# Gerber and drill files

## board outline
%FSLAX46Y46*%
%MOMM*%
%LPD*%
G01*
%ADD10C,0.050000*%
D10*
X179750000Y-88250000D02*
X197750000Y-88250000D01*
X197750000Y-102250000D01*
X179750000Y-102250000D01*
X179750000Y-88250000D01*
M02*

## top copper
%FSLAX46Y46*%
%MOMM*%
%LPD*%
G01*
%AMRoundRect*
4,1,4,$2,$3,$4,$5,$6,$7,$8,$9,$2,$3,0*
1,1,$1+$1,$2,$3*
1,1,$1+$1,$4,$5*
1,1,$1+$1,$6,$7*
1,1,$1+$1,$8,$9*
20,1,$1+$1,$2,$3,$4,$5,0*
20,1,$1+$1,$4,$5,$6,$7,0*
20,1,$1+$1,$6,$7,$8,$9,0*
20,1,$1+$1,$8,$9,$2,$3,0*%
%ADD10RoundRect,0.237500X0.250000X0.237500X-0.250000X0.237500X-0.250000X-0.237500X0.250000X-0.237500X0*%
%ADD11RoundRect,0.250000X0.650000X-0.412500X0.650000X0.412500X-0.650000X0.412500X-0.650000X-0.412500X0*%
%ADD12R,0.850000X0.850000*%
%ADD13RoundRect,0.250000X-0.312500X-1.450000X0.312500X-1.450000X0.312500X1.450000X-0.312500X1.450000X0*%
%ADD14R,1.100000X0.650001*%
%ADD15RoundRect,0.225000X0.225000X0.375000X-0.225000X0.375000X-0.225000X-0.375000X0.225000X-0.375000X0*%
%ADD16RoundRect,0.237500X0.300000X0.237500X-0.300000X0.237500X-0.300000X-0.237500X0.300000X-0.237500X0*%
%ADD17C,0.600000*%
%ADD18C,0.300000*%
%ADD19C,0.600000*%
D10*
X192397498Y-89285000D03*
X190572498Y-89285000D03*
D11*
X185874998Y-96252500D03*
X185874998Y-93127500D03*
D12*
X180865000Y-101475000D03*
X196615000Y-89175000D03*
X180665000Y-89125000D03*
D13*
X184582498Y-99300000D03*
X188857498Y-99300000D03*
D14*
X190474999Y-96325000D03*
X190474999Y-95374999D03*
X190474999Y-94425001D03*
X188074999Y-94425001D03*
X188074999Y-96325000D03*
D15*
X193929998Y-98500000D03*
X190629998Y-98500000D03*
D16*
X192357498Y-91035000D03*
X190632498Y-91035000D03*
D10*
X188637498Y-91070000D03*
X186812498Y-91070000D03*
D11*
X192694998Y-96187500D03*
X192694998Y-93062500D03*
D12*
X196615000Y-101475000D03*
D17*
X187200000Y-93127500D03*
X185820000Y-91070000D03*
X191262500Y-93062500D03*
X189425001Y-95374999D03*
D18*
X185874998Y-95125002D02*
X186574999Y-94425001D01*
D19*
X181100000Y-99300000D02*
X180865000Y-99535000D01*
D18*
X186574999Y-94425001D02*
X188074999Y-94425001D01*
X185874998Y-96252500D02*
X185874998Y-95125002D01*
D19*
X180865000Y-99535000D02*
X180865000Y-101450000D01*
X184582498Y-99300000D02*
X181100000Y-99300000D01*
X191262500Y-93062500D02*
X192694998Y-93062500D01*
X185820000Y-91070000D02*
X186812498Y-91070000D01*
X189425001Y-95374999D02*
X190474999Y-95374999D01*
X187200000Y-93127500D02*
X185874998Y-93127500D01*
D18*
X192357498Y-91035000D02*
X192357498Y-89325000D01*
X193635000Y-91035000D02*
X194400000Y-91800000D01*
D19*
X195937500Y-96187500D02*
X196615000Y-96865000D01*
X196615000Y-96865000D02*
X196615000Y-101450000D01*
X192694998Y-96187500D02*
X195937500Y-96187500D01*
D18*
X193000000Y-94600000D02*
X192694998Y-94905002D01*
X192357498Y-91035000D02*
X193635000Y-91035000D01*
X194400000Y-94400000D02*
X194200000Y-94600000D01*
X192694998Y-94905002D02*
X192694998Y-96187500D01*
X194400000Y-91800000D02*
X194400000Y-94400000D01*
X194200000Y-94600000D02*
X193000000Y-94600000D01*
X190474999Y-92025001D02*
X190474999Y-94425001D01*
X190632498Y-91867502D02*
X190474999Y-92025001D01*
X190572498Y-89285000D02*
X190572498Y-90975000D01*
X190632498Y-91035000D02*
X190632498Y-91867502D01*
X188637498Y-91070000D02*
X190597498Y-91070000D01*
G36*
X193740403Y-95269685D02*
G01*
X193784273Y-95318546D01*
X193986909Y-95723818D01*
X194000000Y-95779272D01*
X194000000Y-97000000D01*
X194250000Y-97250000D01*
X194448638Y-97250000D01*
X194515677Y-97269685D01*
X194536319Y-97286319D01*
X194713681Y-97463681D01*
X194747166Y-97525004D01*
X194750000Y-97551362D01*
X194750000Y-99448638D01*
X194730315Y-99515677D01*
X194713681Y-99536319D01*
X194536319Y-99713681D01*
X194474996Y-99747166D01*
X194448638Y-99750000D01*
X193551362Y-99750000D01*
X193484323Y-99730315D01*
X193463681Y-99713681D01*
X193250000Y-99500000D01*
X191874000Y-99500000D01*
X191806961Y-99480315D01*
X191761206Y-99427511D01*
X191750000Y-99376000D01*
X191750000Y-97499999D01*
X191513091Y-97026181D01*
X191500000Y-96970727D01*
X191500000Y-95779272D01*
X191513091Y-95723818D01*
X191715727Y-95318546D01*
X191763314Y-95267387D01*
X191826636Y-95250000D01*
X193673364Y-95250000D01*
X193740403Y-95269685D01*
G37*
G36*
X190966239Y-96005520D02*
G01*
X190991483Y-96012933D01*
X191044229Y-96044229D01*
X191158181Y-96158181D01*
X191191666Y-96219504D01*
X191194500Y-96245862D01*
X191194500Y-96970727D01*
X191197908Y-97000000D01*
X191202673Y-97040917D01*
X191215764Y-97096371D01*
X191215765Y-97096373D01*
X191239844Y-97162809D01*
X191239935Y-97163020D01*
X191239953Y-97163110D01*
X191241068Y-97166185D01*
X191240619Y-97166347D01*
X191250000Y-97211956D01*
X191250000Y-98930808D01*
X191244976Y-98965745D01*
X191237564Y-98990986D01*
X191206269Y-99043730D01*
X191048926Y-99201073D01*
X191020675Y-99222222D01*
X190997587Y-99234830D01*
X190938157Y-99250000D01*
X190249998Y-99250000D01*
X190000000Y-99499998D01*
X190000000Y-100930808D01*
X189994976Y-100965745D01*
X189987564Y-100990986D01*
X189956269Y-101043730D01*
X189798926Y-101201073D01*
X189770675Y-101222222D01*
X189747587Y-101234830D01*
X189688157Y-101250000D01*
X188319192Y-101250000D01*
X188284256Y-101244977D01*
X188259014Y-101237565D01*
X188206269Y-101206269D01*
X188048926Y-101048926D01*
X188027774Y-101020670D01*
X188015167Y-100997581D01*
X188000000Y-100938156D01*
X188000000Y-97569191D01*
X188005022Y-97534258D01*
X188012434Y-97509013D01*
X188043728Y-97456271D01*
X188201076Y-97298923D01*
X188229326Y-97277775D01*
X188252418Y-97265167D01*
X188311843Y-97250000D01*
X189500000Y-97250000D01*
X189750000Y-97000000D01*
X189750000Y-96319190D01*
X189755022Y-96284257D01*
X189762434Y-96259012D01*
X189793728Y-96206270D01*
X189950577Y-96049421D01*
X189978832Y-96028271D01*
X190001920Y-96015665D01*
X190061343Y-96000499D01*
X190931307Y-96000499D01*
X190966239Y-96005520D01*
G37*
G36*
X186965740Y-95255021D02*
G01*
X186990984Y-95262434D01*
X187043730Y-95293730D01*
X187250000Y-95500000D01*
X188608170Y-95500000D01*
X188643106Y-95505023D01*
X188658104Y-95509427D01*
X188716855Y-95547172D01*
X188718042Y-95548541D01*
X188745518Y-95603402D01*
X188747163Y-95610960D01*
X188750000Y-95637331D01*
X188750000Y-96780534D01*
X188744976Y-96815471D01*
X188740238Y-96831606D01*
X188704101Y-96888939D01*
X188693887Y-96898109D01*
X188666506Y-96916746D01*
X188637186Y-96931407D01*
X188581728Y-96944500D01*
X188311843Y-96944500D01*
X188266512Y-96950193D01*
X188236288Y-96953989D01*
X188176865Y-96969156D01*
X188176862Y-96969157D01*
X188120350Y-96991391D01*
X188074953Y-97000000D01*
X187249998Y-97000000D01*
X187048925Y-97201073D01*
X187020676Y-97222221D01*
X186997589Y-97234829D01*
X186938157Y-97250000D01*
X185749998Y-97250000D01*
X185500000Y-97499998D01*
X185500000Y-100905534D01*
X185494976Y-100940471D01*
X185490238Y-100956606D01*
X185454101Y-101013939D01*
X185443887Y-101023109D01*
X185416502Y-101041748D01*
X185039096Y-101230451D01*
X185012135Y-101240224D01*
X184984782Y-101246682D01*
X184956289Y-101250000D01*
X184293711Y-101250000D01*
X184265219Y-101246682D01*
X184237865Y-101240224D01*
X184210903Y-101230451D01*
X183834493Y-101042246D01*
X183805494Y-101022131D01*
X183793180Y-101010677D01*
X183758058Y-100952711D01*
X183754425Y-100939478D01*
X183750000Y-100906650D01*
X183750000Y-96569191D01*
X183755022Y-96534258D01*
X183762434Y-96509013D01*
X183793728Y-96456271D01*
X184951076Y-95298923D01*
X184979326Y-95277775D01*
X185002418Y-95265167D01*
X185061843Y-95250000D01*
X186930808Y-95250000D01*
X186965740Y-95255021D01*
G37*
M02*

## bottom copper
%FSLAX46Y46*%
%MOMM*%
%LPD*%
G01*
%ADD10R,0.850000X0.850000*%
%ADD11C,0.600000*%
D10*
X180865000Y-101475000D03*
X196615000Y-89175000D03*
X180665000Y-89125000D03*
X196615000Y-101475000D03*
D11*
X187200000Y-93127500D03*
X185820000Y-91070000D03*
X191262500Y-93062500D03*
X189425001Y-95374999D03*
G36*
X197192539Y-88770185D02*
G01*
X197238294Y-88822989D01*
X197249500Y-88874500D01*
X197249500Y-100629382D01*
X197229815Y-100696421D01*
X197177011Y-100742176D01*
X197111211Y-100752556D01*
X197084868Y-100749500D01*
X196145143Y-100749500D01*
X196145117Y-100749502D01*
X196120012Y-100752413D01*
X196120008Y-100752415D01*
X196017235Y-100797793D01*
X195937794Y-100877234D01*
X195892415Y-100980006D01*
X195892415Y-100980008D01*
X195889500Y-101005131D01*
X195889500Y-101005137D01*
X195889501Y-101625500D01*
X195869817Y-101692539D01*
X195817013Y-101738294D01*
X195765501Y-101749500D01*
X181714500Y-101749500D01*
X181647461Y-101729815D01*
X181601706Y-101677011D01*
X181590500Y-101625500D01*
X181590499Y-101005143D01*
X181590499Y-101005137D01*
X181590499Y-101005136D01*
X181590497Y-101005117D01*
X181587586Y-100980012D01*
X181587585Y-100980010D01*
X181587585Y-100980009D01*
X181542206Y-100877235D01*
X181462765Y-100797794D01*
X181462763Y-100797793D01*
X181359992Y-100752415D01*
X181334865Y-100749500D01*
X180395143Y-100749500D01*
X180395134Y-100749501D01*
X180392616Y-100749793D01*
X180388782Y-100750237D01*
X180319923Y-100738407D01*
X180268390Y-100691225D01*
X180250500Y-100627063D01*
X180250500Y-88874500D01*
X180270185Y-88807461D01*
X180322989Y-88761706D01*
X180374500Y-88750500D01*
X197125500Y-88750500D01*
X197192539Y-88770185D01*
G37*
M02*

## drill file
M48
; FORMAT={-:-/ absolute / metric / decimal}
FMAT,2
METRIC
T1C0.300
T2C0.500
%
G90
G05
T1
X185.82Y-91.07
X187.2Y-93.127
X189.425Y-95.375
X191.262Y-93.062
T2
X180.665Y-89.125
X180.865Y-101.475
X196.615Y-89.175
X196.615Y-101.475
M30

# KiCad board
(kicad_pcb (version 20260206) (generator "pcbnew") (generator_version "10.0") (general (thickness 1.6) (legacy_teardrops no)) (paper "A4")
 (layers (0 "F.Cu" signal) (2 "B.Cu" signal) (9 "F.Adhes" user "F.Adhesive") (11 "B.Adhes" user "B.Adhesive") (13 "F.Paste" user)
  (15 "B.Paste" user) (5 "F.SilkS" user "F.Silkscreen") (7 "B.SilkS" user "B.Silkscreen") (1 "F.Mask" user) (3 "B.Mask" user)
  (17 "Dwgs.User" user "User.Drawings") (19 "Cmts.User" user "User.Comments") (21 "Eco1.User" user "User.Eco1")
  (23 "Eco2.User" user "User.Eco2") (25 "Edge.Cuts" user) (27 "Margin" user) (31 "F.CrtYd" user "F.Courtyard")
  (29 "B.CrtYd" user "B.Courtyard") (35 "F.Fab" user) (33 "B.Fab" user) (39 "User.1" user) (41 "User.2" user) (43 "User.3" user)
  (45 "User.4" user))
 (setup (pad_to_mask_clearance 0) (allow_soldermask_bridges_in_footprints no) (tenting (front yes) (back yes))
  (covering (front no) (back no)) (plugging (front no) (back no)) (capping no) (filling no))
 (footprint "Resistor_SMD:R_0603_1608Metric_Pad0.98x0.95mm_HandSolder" (layer "F.Cu") (at 191.484998 89.285 180)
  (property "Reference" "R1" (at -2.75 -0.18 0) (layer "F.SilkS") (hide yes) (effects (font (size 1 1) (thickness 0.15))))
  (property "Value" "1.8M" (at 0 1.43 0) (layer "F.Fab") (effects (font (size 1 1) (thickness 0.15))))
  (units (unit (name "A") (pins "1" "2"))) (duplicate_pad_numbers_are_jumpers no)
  (pad "1" smd roundrect (at -0.9125 0 180) (size 0.975 0.95) (layers "F.Cu" "F.Mask" "F.Paste") (roundrect_rratio 0.25) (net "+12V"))
  (pad "2" smd roundrect (at 0.9125 0 180) (size 0.975 0.95) (layers "F.Cu" "F.Mask" "F.Paste") (roundrect_rratio 0.25) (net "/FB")))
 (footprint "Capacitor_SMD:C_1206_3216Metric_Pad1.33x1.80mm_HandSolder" (layer "F.Cu") (at 185.874998 94.69 90)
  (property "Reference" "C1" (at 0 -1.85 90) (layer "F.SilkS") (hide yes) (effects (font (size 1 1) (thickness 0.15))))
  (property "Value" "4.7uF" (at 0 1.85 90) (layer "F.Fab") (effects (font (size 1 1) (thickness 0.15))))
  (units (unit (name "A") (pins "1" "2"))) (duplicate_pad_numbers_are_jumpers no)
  (pad "1" smd roundrect (at -1.5625 0 90) (size 1.325 1.8) (layers "F.Cu" "F.Mask" "F.Paste") (roundrect_rratio 0.188679) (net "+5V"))
  (pad "2" smd roundrect (at 1.5625 0 90) (size 1.325 1.8) (layers "F.Cu" "F.Mask" "F.Paste") (roundrect_rratio 0.188679) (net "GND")))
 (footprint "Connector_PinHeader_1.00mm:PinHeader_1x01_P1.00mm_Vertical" (layer "F.Cu") (at 180.865 101.475)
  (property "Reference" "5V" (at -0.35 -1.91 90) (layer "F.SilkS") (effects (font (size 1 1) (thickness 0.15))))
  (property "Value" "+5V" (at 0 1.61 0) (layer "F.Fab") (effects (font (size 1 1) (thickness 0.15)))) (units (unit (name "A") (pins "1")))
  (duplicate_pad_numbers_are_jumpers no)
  (pad "1" thru_hole rect (at 0 0) (size 0.85 0.85) (drill 0.5) (layers "*.Cu" "*.Mask") (remove_unused_layers no) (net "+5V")))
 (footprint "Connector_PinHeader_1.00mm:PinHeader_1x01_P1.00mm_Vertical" (layer "F.Cu") (at 196.615 89.175)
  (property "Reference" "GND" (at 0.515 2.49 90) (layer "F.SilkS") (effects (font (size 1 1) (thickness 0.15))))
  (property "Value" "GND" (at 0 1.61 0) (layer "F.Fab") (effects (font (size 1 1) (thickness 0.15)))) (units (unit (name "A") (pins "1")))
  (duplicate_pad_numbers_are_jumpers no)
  (pad "1" thru_hole rect (at 0 0) (size 0.85 0.85) (drill 0.5) (layers "*.Cu" "*.Mask") (remove_unused_layers no) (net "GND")))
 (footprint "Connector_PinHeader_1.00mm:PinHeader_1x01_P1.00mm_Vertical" (layer "F.Cu") (at 180.665 89.125)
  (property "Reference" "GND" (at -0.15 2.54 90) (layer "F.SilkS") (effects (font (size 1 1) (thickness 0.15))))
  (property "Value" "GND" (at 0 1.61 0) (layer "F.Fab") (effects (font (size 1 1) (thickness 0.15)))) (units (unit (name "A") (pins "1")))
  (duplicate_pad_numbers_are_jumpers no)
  (pad "1" thru_hole rect (at 0 0) (size 0.85 0.85) (drill 0.5) (layers "*.Cu" "*.Mask") (remove_unused_layers no) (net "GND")))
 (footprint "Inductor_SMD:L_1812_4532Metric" (layer "F.Cu") (at 186.719998 99.3)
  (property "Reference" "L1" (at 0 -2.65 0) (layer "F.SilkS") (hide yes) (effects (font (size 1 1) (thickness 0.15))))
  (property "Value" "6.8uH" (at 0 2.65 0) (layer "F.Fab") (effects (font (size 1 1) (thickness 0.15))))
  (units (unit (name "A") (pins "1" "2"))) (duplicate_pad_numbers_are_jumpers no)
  (pad "1" smd roundrect (at -2.1375 0) (size 1.125 3.4) (layers "F.Cu" "F.Mask" "F.Paste") (roundrect_rratio 0.222222) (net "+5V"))
  (pad "2" smd roundrect (at 2.1375 0) (size 1.125 3.4) (layers "F.Cu" "F.Mask" "F.Paste") (roundrect_rratio 0.222222) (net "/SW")))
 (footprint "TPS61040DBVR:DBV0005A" (layer "F.Cu") (at 189.274999 95.374999 180)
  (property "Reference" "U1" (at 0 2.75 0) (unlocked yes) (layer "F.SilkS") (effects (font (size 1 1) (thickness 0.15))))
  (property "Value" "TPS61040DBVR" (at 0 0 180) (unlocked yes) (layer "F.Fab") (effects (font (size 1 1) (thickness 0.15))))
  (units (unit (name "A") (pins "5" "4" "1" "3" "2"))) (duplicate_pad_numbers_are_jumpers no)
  (pad "1" smd rect (at -1.2 -0.950001 270) (size 0.650001 1.1) (layers "F.Cu" "F.Mask" "F.Paste") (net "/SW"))
  (pad "2" smd rect (at -1.2 0 270) (size 0.650001 1.1) (layers "F.Cu" "F.Mask" "F.Paste") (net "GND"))
  (pad "3" smd rect (at -1.2 0.949998 270) (size 0.650001 1.1) (layers "F.Cu" "F.Mask" "F.Paste") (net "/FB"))
  (pad "4" smd rect (at 1.2 0.949998 270) (size 0.650001 1.1) (layers "F.Cu" "F.Mask" "F.Paste") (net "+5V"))
  (pad "5" smd rect (at 1.2 -0.950001 270) (size 0.650001 1.1) (layers "F.Cu" "F.Mask" "F.Paste") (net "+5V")))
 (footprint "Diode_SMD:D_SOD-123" (layer "F.Cu") (at 192.279998 98.5 180)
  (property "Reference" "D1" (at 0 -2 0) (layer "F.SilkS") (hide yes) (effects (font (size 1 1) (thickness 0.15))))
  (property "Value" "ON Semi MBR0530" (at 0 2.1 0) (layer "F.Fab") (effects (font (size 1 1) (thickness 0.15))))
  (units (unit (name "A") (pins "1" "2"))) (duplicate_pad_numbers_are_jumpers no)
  (pad "1" smd roundrect (at -1.65 0 180) (size 0.9 1.2) (layers "F.Cu" "F.Mask" "F.Paste") (roundrect_rratio 0.25) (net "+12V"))
  (pad "2" smd roundrect (at 1.65 0 180) (size 0.9 1.2) (layers "F.Cu" "F.Mask" "F.Paste") (roundrect_rratio 0.25) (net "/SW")))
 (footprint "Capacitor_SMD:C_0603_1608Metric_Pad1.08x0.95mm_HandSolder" (layer "F.Cu") (at 191.494998 91.035 180)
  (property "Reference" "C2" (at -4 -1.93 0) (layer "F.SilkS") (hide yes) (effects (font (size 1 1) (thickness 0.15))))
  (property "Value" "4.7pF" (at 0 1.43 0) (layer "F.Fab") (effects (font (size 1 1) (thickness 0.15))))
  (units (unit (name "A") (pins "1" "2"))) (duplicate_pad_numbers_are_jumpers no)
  (pad "1" smd roundrect (at -0.8625 0 180) (size 1.075 0.95) (layers "F.Cu" "F.Mask" "F.Paste") (roundrect_rratio 0.25) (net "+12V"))
  (pad "2" smd roundrect (at 0.8625 0 180) (size 1.075 0.95) (layers "F.Cu" "F.Mask" "F.Paste") (roundrect_rratio 0.25) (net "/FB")))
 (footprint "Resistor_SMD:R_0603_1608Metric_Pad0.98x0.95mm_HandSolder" (layer "F.Cu") (at 187.724998 91.07 180)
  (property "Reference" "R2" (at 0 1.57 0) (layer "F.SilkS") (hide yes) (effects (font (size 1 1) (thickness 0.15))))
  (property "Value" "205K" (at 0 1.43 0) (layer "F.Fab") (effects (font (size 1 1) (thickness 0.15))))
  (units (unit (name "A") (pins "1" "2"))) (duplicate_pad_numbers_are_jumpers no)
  (pad "1" smd roundrect (at -0.9125 0 180) (size 0.975 0.95) (layers "F.Cu" "F.Mask" "F.Paste") (roundrect_rratio 0.25) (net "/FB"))
  (pad "2" smd roundrect (at 0.9125 0 180) (size 0.975 0.95) (layers "F.Cu" "F.Mask" "F.Paste") (roundrect_rratio 0.25) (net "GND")))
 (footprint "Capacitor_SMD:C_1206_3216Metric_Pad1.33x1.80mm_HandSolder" (layer "F.Cu") (at 192.694998 94.625 90)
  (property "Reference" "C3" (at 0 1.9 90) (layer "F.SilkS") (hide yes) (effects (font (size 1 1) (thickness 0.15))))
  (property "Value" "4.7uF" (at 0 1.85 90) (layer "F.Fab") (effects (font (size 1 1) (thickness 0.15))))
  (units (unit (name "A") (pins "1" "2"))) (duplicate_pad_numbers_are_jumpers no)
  (pad "1" smd roundrect (at -1.5625 0 90) (size 1.325 1.8) (layers "F.Cu" "F.Mask" "F.Paste") (roundrect_rratio 0.188679) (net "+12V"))
  (pad "2" smd roundrect (at 1.5625 0 90) (size 1.325 1.8) (layers "F.Cu" "F.Mask" "F.Paste") (roundrect_rratio 0.188679) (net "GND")))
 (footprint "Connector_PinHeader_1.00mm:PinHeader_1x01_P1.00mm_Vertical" (layer "F.Cu") (at 196.615 101.475)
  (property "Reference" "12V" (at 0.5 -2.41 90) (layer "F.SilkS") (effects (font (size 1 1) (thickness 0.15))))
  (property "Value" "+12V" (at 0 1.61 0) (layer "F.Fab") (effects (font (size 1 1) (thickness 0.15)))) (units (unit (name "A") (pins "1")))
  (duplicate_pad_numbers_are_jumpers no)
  (pad "1" thru_hole rect (at 0 0) (size 0.85 0.85) (drill 0.5) (layers "*.Cu" "*.Mask") (remove_unused_layers no) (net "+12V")))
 (gr_rect (start 179.75 88.25) (end 197.75 102.25) (stroke (width 0.05) (type default)) (fill no) (layer "Edge.Cuts"))
 (segment (start 185.874998 95.125002) (end 186.574999 94.425001) (width 0.3) (layer "F.Cu") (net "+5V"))
 (segment (start 181.1 99.3) (end 180.865 99.535) (width 0.6) (layer "F.Cu") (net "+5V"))
 (segment (start 186.574999 94.425001) (end 188.074999 94.425001) (width 0.3) (layer "F.Cu") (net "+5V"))
 (segment (start 185.874998 96.2525) (end 185.874998 95.125002) (width 0.3) (layer "F.Cu") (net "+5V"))
 (segment (start 180.865 99.535) (end 180.865 101.45) (width 0.6) (layer "F.Cu") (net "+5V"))
 (segment (start 184.582498 99.3) (end 181.1 99.3) (width 0.6) (layer "F.Cu") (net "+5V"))
 (segment (start 191.2625 93.0625) (end 192.694998 93.0625) (width 0.6) (layer "F.Cu") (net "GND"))
 (segment (start 185.82 91.07) (end 186.812498 91.07) (width 0.6) (layer "F.Cu") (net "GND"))
 (segment (start 189.425001 95.374999) (end 190.474999 95.374999) (width 0.6) (layer "F.Cu") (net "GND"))
 (segment (start 187.2 93.1275) (end 185.874998 93.1275) (width 0.6) (layer "F.Cu") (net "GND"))
 (via (at 187.2 93.1275) (size 0.6) (drill 0.3) (layers "F.Cu" "B.Cu") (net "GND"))
 (via (at 185.82 91.07) (size 0.6) (drill 0.3) (layers "F.Cu" "B.Cu") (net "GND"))
 (via (at 191.2625 93.0625) (size 0.6) (drill 0.3) (layers "F.Cu" "B.Cu") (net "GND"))
 (via (at 189.425001 95.374999) (size 0.6) (drill 0.3) (layers "F.Cu" "B.Cu") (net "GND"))
 (segment (start 192.357498 91.035) (end 192.357498 89.325) (width 0.3) (layer "F.Cu") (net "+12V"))
 (segment (start 193.635 91.035) (end 194.4 91.8) (width 0.3) (layer "F.Cu") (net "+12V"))
 (segment (start 195.9375 96.1875) (end 196.615 96.865) (width 0.6) (layer "F.Cu") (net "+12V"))
 (segment (start 196.615 96.865) (end 196.615 101.45) (width 0.6) (layer "F.Cu") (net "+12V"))
 (segment (start 192.694998 96.1875) (end 195.9375 96.1875) (width 0.6) (layer "F.Cu") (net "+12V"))
 (segment (start 193 94.6) (end 192.694998 94.905002) (width 0.3) (layer "F.Cu") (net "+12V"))
 (segment (start 192.357498 91.035) (end 193.635 91.035) (width 0.3) (layer "F.Cu") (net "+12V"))
 (segment (start 194.4 94.4) (end 194.2 94.6) (width 0.3) (layer "F.Cu") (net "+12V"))
 (segment (start 192.694998 94.905002) (end 192.694998 96.1875) (width 0.3) (layer "F.Cu") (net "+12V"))
 (segment (start 194.4 91.8) (end 194.4 94.4) (width 0.3) (layer "F.Cu") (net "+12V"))
 (segment (start 194.2 94.6) (end 193 94.6) (width 0.3) (layer "F.Cu") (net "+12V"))
 (segment (start 190.474999 92.025001) (end 190.474999 94.425001) (width 0.3) (layer "F.Cu") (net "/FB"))
 (segment (start 190.632498 91.867502) (end 190.474999 92.025001) (width 0.3) (layer "F.Cu") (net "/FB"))
 (segment (start 190.572498 89.285) (end 190.572498 90.975) (width 0.3) (layer "F.Cu") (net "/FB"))
 (segment (start 190.632498 91.035) (end 190.632498 91.867502) (width 0.3) (layer "F.Cu") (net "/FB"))
 (segment (start 188.637498 91.07) (end 190.597498 91.07) (width 0.3) (layer "F.Cu") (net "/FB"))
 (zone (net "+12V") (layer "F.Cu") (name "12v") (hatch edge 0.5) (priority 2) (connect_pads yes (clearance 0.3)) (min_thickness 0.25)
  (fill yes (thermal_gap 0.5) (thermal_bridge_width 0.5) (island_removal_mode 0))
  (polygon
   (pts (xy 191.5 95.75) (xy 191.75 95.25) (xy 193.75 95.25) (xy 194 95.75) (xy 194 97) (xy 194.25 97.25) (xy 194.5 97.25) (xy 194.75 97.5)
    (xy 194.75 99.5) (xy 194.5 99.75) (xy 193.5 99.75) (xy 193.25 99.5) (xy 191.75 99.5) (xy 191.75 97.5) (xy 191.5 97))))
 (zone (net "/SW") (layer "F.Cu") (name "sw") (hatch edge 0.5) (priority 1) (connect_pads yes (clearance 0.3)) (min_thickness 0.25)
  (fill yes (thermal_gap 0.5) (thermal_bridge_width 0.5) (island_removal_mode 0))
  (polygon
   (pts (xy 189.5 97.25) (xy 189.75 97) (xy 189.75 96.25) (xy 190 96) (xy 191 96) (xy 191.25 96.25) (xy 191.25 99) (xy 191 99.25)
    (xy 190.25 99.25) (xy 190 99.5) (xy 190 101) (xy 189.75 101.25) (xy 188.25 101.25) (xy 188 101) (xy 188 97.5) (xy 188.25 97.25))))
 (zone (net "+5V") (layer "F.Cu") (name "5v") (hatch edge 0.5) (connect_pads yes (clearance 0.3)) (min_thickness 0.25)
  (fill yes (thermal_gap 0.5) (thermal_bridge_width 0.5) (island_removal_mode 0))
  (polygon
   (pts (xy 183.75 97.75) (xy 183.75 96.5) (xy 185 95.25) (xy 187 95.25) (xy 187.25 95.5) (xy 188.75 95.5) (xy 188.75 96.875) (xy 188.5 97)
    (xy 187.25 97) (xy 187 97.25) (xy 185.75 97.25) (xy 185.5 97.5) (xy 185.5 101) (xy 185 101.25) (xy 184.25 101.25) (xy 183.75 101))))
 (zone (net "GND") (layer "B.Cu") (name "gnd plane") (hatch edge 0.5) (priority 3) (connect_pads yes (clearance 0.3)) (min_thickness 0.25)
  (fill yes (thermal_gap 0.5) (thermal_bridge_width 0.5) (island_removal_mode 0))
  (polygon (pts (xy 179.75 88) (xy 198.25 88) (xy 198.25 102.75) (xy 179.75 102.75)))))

